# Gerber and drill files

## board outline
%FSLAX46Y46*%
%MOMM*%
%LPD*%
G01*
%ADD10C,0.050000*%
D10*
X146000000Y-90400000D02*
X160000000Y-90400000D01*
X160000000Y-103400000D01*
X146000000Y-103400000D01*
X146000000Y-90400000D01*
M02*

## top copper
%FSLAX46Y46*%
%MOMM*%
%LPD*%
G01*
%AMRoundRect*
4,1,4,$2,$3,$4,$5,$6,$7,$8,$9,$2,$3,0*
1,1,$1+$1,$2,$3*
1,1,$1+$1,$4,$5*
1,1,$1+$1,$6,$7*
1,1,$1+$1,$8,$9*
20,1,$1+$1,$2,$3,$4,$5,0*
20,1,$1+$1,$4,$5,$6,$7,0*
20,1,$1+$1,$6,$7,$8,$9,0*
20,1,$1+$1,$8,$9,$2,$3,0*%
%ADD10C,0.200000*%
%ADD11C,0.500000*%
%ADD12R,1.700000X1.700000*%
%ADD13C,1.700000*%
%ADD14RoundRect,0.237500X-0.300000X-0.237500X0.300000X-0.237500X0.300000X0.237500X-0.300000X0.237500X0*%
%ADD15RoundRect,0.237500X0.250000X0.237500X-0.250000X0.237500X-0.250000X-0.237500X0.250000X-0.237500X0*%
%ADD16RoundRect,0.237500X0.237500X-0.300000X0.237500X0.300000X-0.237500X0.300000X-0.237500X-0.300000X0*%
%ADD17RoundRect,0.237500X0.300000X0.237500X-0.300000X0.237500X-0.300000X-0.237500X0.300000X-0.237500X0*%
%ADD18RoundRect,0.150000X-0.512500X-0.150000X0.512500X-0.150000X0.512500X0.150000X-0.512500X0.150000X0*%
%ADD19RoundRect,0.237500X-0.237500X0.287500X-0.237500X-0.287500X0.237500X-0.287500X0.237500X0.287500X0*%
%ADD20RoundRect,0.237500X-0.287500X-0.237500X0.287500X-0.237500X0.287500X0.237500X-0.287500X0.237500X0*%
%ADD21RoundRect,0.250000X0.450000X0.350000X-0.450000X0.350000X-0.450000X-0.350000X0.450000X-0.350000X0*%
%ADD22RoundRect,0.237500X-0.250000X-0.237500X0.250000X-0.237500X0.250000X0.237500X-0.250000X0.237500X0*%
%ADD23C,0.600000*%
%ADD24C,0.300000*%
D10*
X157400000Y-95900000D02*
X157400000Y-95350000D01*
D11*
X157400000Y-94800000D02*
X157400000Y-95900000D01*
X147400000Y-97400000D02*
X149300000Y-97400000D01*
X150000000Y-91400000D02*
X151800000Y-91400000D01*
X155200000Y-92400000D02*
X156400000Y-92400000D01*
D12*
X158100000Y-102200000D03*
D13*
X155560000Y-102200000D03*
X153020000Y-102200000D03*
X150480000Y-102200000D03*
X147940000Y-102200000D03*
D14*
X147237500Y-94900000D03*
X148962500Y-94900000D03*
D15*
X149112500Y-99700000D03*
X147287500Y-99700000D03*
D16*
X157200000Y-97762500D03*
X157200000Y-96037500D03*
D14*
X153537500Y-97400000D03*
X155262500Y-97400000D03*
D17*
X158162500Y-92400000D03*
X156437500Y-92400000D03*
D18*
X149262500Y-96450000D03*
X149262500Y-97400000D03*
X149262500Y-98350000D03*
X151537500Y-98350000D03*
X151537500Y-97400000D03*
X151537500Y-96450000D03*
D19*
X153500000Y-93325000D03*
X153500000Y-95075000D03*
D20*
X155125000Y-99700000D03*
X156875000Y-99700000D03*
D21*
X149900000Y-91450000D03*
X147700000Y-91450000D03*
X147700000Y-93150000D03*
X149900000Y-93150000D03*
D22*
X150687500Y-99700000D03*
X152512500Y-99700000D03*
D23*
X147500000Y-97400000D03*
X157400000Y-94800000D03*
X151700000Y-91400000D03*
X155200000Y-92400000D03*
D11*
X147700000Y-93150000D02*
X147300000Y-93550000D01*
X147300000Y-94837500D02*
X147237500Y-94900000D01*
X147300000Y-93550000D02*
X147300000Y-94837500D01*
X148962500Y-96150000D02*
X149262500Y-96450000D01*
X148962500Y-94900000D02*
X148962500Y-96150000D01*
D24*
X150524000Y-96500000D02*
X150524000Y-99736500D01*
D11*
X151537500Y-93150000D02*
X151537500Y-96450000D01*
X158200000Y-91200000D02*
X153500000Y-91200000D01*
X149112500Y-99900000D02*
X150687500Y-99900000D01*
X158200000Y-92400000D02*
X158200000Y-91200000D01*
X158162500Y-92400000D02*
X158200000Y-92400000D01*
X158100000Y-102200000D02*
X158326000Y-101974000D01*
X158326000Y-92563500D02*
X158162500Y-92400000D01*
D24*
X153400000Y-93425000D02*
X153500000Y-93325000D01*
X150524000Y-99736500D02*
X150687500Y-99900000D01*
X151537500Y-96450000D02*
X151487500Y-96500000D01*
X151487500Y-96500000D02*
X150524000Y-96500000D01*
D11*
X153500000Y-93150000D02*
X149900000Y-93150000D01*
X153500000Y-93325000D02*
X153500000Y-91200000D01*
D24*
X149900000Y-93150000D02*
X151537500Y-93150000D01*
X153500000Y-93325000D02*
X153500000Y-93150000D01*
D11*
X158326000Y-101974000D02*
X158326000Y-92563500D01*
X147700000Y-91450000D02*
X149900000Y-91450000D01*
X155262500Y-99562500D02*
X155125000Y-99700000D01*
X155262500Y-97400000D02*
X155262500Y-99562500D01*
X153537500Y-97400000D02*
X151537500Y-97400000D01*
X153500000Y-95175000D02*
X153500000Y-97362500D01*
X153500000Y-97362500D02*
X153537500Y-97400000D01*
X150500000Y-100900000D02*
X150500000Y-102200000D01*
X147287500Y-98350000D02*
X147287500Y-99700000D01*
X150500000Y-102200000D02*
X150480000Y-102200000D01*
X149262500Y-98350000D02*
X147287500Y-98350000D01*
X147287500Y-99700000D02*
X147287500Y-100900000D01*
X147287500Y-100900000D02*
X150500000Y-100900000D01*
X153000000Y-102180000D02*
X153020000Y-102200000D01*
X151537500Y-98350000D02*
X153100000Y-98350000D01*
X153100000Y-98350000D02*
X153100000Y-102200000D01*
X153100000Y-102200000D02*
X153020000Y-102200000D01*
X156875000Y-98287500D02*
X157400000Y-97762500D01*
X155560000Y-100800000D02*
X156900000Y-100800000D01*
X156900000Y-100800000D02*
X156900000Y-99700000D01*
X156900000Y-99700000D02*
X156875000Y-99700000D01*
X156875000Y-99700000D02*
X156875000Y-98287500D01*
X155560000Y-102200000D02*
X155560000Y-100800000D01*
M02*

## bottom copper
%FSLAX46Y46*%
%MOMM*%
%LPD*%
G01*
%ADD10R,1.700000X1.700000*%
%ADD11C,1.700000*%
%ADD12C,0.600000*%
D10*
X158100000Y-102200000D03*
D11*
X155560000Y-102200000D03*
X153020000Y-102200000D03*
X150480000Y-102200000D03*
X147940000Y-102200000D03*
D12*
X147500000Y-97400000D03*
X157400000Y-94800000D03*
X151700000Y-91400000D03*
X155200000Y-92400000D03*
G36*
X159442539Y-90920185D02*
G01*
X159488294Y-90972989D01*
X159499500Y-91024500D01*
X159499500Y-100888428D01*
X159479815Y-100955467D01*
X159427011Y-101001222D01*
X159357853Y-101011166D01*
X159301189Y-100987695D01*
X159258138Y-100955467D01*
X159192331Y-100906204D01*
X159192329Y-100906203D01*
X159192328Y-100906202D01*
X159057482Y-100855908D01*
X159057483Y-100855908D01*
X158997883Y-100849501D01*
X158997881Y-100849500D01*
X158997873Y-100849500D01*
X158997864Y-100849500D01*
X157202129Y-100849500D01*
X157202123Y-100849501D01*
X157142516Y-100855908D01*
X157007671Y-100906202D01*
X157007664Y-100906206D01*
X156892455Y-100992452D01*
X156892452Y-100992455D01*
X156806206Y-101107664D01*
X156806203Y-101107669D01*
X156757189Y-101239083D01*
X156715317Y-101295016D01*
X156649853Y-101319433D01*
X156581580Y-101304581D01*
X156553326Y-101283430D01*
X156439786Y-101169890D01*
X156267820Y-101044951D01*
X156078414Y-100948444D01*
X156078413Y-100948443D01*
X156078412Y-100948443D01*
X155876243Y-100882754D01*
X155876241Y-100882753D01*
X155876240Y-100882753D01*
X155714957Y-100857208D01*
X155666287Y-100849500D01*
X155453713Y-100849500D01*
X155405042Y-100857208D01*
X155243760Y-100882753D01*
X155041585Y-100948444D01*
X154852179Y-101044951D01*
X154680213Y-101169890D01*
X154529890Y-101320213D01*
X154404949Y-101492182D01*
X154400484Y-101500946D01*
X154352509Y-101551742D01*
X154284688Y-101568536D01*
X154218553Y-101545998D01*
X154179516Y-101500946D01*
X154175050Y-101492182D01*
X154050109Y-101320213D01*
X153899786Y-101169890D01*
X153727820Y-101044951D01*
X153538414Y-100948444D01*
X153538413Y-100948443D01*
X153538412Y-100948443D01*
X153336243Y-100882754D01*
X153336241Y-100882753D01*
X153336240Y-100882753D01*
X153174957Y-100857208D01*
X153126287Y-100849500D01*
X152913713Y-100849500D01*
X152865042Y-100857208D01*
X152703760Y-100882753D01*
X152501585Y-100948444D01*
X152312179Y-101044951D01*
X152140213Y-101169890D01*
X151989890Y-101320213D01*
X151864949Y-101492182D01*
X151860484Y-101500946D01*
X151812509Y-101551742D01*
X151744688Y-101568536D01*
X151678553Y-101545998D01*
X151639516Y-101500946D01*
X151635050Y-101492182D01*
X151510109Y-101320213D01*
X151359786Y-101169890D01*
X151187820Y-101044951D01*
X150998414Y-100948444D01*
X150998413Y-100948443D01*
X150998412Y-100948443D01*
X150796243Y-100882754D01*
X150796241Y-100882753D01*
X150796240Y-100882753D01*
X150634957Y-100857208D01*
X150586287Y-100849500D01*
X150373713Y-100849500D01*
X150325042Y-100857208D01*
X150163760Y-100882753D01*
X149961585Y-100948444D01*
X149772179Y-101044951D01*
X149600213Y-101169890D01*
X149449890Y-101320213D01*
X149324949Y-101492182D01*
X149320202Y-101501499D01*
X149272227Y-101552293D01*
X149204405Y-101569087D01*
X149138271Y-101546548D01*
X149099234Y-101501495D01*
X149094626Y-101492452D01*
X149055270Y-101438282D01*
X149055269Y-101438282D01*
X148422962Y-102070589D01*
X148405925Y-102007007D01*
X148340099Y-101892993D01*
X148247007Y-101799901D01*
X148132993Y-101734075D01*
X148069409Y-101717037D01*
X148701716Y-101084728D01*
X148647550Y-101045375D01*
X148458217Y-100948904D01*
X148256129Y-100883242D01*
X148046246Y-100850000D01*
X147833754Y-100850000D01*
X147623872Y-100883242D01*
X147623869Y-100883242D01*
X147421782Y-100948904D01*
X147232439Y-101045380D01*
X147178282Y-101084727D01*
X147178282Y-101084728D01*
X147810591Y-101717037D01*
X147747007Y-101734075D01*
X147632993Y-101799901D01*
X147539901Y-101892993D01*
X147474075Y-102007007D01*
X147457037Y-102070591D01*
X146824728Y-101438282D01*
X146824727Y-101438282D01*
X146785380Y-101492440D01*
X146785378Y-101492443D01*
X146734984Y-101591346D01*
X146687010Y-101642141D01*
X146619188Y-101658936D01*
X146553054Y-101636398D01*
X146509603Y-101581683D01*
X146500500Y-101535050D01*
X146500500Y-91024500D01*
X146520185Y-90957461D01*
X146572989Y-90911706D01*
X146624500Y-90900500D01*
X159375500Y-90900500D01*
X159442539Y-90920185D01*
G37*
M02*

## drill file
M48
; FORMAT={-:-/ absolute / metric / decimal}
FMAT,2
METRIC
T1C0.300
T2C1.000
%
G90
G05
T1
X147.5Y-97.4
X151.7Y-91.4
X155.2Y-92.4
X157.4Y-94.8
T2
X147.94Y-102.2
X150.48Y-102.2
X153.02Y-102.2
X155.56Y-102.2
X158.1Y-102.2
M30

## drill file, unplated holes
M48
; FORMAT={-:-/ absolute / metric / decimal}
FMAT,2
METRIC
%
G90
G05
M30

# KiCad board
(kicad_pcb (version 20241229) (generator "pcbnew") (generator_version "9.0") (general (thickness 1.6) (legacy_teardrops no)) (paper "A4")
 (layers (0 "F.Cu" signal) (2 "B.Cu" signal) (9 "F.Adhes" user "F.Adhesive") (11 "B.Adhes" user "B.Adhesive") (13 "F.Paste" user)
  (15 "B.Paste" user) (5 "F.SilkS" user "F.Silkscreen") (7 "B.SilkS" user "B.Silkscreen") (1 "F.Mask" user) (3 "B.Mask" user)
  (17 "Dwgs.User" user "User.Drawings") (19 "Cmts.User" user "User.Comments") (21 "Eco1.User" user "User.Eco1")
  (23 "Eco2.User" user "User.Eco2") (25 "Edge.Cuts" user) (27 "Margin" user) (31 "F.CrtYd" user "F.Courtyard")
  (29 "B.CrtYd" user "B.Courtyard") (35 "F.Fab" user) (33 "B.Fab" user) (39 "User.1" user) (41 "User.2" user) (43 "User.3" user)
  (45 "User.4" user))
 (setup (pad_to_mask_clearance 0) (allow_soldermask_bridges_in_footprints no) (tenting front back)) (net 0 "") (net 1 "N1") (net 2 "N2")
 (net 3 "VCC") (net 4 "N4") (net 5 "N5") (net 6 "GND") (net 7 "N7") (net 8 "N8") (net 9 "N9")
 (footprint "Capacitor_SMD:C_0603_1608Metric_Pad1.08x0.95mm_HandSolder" (layer "F.Cu") (at 148.1 94.9)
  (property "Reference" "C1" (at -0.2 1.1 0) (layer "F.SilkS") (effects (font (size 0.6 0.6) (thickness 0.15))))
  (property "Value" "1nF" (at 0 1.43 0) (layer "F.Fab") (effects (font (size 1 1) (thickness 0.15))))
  (pad "1" smd roundrect (at -0.8625 0) (size 1.075 0.95) (layers "F.Cu" "F.Mask" "F.Paste") (roundrect_rratio 0.25) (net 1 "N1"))
  (pad "2" smd roundrect (at 0.8625 0) (size 1.075 0.95) (layers "F.Cu" "F.Mask" "F.Paste") (roundrect_rratio 0.25) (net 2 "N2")))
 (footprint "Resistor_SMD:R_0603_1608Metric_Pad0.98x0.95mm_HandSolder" (layer "F.Cu") (at 148.2 99.7 180)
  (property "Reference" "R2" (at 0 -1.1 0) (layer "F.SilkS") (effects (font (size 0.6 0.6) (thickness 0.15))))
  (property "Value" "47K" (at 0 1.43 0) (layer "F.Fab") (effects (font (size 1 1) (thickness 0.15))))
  (pad "1" smd roundrect (at -0.9125 0 180) (size 0.975 0.95) (layers "F.Cu" "F.Mask" "F.Paste") (roundrect_rratio 0.25) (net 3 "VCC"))
  (pad "2" smd roundrect (at 0.9125 0 180) (size 0.975 0.95) (layers "F.Cu" "F.Mask" "F.Paste") (roundrect_rratio 0.25) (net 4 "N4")))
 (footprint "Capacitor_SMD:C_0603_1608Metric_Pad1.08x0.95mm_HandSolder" (layer "F.Cu") (at 157.2 96.9 90)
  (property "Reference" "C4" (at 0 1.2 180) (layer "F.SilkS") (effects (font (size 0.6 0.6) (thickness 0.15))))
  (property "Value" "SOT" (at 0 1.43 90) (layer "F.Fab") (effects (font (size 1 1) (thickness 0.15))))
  (pad "1" smd roundrect (at -0.8625 0 90) (size 1.075 0.95) (layers "F.Cu" "F.Mask" "F.Paste") (roundrect_rratio 0.25) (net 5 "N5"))
  (pad "2" smd roundrect (at 0.8625 0 90) (size 1.075 0.95) (layers "F.Cu" "F.Mask" "F.Paste") (roundrect_rratio 0.25) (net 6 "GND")))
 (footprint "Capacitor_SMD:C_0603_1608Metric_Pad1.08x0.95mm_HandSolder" (layer "F.Cu") (at 154.4 97.4)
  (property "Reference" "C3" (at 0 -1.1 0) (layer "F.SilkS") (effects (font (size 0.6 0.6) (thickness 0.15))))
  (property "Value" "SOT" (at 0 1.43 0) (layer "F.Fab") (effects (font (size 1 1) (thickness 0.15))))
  (pad "1" smd roundrect (at -0.8625 0) (size 1.075 0.95) (layers "F.Cu" "F.Mask" "F.Paste") (roundrect_rratio 0.25) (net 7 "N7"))
  (pad "2" smd roundrect (at 0.8625 0) (size 1.075 0.95) (layers "F.Cu" "F.Mask" "F.Paste") (roundrect_rratio 0.25) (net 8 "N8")))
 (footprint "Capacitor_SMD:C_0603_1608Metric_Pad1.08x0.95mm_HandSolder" (layer "F.Cu") (at 157.3 92.4 180)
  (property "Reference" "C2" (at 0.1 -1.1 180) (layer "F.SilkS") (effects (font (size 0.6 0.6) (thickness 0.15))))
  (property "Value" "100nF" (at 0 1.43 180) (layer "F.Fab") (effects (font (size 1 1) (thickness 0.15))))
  (pad "1" smd roundrect (at -0.8625 0 180) (size 1.075 0.95) (layers "F.Cu" "F.Mask" "F.Paste") (roundrect_rratio 0.25) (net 3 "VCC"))
  (pad "2" smd roundrect (at 0.8625 0 180) (size 1.075 0.95) (layers "F.Cu" "F.Mask" "F.Paste") (roundrect_rratio 0.25) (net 6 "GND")))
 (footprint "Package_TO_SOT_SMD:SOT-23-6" (layer "F.Cu") (at 150.4 97.4)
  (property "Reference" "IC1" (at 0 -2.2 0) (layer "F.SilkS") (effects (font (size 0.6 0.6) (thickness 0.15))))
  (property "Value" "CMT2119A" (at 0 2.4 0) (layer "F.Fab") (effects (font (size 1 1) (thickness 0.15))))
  (pad "1" smd roundrect (at -1.1375 -0.95) (size 1.325 0.6) (layers "F.Cu" "F.Mask" "F.Paste") (roundrect_rratio 0.25) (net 2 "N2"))
  (pad "2" smd roundrect (at -1.1375 0) (size 1.325 0.6) (layers "F.Cu" "F.Mask" "F.Paste") (roundrect_rratio 0.25) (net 6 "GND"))
  (pad "3" smd roundrect (at -1.1375 0.95) (size 1.325 0.6) (layers "F.Cu" "F.Mask" "F.Paste") (roundrect_rratio 0.25) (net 4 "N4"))
  (pad "4" smd roundrect (at 1.1375 0.95) (size 1.325 0.6) (layers "F.Cu" "F.Mask" "F.Paste") (roundrect_rratio 0.25) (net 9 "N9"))
  (pad "5" smd roundrect (at 1.1375 0) (size 1.325 0.6) (layers "F.Cu" "F.Mask" "F.Paste") (roundrect_rratio 0.25) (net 7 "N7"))
  (pad "6" smd roundrect (at 1.1375 -0.95) (size 1.325 0.6) (layers "F.Cu" "F.Mask" "F.Paste") (roundrect_rratio 0.25) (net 3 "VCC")))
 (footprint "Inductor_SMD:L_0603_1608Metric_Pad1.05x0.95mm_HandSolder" (layer "F.Cu") (at 153.5 94.2 -90)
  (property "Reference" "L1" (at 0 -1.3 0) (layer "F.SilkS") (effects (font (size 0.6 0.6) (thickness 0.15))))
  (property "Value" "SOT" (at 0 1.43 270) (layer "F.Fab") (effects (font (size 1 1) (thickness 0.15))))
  (pad "1" smd roundrect (at -0.875 0 270) (size 1.05 0.95) (layers "F.Cu" "F.Mask" "F.Paste") (roundrect_rratio 0.25) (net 3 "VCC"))
  (pad "2" smd roundrect (at 0.875 0 270) (size 1.05 0.95) (layers "F.Cu" "F.Mask" "F.Paste") (roundrect_rratio 0.25) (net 7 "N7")))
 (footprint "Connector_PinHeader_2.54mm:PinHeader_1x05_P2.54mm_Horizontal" (layer "F.Cu") (at 158.1 102.2 -90)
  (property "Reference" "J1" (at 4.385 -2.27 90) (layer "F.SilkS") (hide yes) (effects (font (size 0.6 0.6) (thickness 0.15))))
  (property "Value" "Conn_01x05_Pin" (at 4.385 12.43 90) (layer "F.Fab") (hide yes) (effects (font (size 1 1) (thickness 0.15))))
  (pad "1" thru_hole rect (at 0 0 270) (size 1.7 1.7) (drill 1) (layers "*.Cu" "*.Mask") (remove_unused_layers no) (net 3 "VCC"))
  (pad "2" thru_hole circle (at 0 2.54 270) (size 1.7 1.7) (drill 1) (layers "*.Cu" "*.Mask") (remove_unused_layers no) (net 5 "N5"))
  (pad "3" thru_hole circle (at 0 5.08 270) (size 1.7 1.7) (drill 1) (layers "*.Cu" "*.Mask") (remove_unused_layers no) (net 9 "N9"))
  (pad "4" thru_hole circle (at 0 7.62 270) (size 1.7 1.7) (drill 1) (layers "*.Cu" "*.Mask") (remove_unused_layers no) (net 4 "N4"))
  (pad "5" thru_hole circle (at 0 10.16 270) (size 1.7 1.7) (drill 1) (layers "*.Cu" "*.Mask") (remove_unused_layers no) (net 6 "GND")))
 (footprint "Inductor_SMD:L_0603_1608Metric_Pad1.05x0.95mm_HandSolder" (layer "F.Cu") (at 156 99.7)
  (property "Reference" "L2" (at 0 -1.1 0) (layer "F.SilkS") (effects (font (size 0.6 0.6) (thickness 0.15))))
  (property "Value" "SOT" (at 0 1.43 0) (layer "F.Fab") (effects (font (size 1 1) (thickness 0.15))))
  (pad "1" smd roundrect (at -0.875 0) (size 1.05 0.95) (layers "F.Cu" "F.Mask" "F.Paste") (roundrect_rratio 0.25) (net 8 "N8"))
  (pad "2" smd roundrect (at 0.875 0) (size 1.05 0.95) (layers "F.Cu" "F.Mask" "F.Paste") (roundrect_rratio 0.25) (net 5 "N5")))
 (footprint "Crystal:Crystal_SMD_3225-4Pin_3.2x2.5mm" (layer "F.Cu") (at 148.8 92.3 180)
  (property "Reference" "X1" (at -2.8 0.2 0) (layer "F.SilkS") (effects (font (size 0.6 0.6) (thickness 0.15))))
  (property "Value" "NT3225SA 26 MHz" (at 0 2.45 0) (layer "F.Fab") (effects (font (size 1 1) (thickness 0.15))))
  (pad "1" smd roundrect (at -1.1 0.85 180) (size 1.4 1.2) (layers "F.Cu" "F.Mask" "F.Paste") (roundrect_rratio 0.208333) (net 6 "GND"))
  (pad "2" smd roundrect (at 1.1 0.85 180) (size 1.4 1.2) (layers "F.Cu" "F.Mask" "F.Paste") (roundrect_rratio 0.208333) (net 6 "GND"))
  (pad "3" smd roundrect (at 1.1 -0.85 180) (size 1.4 1.2) (layers "F.Cu" "F.Mask" "F.Paste") (roundrect_rratio 0.208333) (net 1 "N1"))
  (pad "4" smd roundrect (at -1.1 -0.85 180) (size 1.4 1.2) (layers "F.Cu" "F.Mask" "F.Paste") (roundrect_rratio 0.208333) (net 3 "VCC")))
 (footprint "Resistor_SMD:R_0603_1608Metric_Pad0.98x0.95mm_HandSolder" (layer "F.Cu") (at 151.6 99.7)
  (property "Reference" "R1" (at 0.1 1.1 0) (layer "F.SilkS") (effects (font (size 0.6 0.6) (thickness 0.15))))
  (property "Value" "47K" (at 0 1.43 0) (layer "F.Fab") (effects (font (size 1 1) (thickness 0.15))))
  (pad "1" smd roundrect (at -0.9125 0) (size 0.975 0.95) (layers "F.Cu" "F.Mask" "F.Paste") (roundrect_rratio 0.25) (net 3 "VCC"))
  (pad "2" smd roundrect (at 0.9125 0) (size 0.975 0.95) (layers "F.Cu" "F.Mask" "F.Paste") (roundrect_rratio 0.25) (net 9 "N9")))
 (gr_line (start 157.4 95.9) (end 157.4 95.35) (stroke (width 0.2) (type default)) (layer "F.Cu") (net 6))
 (gr_line (start 157.4 94.8) (end 157.4 95.9) (stroke (width 0.5) (type solid)) (layer "F.Cu") (net 6))
 (gr_line (start 147.4 97.4) (end 149.3 97.4) (stroke (width 0.5) (type solid)) (layer "F.Cu") (net 6))
 (gr_line (start 150 91.4) (end 151.8 91.4) (stroke (width 0.5) (type solid)) (layer "F.Cu") (net 6))
 (gr_line (start 155.2 92.4) (end 156.4 92.4) (stroke (width 0.5) (type solid)) (layer "F.Cu") (net 6))
 (gr_rect (start 146 90.4) (end 160 103.4) (stroke (width 0.05) (type default)) (fill no) (layer "Edge.Cuts"))
 (segment (start 147.7 93.15) (end 147.3 93.55) (width 0.5) (layer "F.Cu") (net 1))
 (segment (start 147.3 94.8375) (end 147.2375 94.9) (width 0.5) (layer "F.Cu") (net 1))
 (segment (start 147.3 93.55) (end 147.3 94.8375) (width 0.5) (layer "F.Cu") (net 1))
 (segment (start 148.9625 96.15) (end 149.2625 96.45) (width 0.5) (layer "F.Cu") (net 2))
 (segment (start 148.9625 94.9) (end 148.9625 96.15) (width 0.5) (layer "F.Cu") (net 2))
 (segment (start 150.524 96.5) (end 150.524 99.7365) (width 0.3) (layer "F.Cu") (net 3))
 (segment (start 151.5375 93.15) (end 151.5375 96.45) (width 0.5) (layer "F.Cu") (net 3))
 (segment (start 158.2 91.2) (end 153.5 91.2) (width 0.5) (layer "F.Cu") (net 3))
 (segment (start 149.1125 99.9) (end 150.6875 99.9) (width 0.5) (layer "F.Cu") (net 3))
 (segment (start 158.2 92.4) (end 158.2 91.2) (width 0.5) (layer "F.Cu") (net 3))
 (segment (start 158.1625 92.4) (end 158.2 92.4) (width 0.5) (layer "F.Cu") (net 3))
 (segment (start 158.1 102.2) (end 158.326 101.974) (width 0.5) (layer "F.Cu") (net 3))
 (segment (start 158.326 92.5635) (end 158.1625 92.4) (width 0.5) (layer "F.Cu") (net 3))
 (segment (start 153.4 93.425) (end 153.5 93.325) (width 0.3) (layer "F.Cu") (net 3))
 (segment (start 150.524 99.7365) (end 150.6875 99.9) (width 0.3) (layer "F.Cu") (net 3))
 (segment (start 151.5375 96.45) (end 151.4875 96.5) (width 0.3) (layer "F.Cu") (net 3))
 (segment (start 151.4875 96.5) (end 150.524 96.5) (width 0.3) (layer "F.Cu") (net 3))
 (segment (start 153.5 93.15) (end 149.9 93.15) (width 0.5) (layer "F.Cu") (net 3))
 (segment (start 153.5 93.325) (end 153.5 91.2) (width 0.5) (layer "F.Cu") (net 3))
 (segment (start 149.9 93.15) (end 151.5375 93.15) (width 0.3) (layer "F.Cu") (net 3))
 (segment (start 153.5 93.325) (end 153.5 93.15) (width 0.3) (layer "F.Cu") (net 3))
 (segment (start 158.326 101.974) (end 158.326 92.5635) (width 0.5) (layer "F.Cu") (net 3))
 (segment (start 147.7 91.45) (end 149.9 91.45) (width 0.5) (layer "F.Cu") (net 6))
 (via (at 147.5 97.4) (size 0.6) (drill 0.3) (layers "F.Cu" "B.Cu") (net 6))
 (via (at 157.4 94.8) (size 0.6) (drill 0.3) (layers "F.Cu" "B.Cu") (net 6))
 (via (at 151.7 91.4) (size 0.6) (drill 0.3) (layers "F.Cu" "B.Cu") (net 6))
 (via (at 155.2 92.4) (size 0.6) (drill 0.3) (layers "F.Cu" "B.Cu") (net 6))
 (segment (start 155.2625 99.5625) (end 155.125 99.7) (width 0.5) (layer "F.Cu") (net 8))
 (segment (start 155.2625 97.4) (end 155.2625 99.5625) (width 0.5) (layer "F.Cu") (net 8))
 (segment (start 153.5375 97.4) (end 151.5375 97.4) (width 0.5) (layer "F.Cu") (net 7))
 (segment (start 153.5 95.175) (end 153.5 97.3625) (width 0.5) (layer "F.Cu") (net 7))
 (segment (start 153.5 97.3625) (end 153.5375 97.4) (width 0.5) (layer "F.Cu") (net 7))
 (segment (start 150.5 100.9) (end 150.5 102.2) (width 0.5) (layer "F.Cu") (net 4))
 (segment (start 147.2875 98.35) (end 147.2875 99.7) (width 0.5) (layer "F.Cu") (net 4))
 (segment (start 150.5 102.2) (end 150.48 102.2) (width 0.5) (layer "F.Cu") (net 4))
 (segment (start 149.2625 98.35) (end 147.2875 98.35) (width 0.5) (layer "F.Cu") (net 4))
 (segment (start 147.2875 99.7) (end 147.2875 100.9) (width 0.5) (layer "F.Cu") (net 4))
 (segment (start 147.2875 100.9) (end 150.5 100.9) (width 0.5) (layer "F.Cu") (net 4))
 (segment (start 153 102.18) (end 153.02 102.2) (width 0.5) (layer "F.Cu") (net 9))
 (segment (start 151.5375 98.35) (end 153.1 98.35) (width 0.5) (layer "F.Cu") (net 9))
 (segment (start 153.1 98.35) (end 153.1 102.2) (width 0.5) (layer "F.Cu") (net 9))
 (segment (start 153.1 102.2) (end 153.02 102.2) (width 0.5) (layer "F.Cu") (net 9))
 (segment (start 156.875 98.2875) (end 157.4 97.7625) (width 0.5) (layer "F.Cu") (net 5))
 (segment (start 155.56 100.8) (end 156.9 100.8) (width 0.5) (layer "F.Cu") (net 5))
 (segment (start 156.9 100.8) (end 156.9 99.7) (width 0.5) (layer "F.Cu") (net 5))
 (segment (start 156.9 99.7) (end 156.875 99.7) (width 0.5) (layer "F.Cu") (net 5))
 (segment (start 156.875 99.7) (end 156.875 98.2875) (width 0.5) (layer "F.Cu") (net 5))
 (segment (start 155.56 102.2) (end 155.56 100.8) (width 0.5) (layer "F.Cu") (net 5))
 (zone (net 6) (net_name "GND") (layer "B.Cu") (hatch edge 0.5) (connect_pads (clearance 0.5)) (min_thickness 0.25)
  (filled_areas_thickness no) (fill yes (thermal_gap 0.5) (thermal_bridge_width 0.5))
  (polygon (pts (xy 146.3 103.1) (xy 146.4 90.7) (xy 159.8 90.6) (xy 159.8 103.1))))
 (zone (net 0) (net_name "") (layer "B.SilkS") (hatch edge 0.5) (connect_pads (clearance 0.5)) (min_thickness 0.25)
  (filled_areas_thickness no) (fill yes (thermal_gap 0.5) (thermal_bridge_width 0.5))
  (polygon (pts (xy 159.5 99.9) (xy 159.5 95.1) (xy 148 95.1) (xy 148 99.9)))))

